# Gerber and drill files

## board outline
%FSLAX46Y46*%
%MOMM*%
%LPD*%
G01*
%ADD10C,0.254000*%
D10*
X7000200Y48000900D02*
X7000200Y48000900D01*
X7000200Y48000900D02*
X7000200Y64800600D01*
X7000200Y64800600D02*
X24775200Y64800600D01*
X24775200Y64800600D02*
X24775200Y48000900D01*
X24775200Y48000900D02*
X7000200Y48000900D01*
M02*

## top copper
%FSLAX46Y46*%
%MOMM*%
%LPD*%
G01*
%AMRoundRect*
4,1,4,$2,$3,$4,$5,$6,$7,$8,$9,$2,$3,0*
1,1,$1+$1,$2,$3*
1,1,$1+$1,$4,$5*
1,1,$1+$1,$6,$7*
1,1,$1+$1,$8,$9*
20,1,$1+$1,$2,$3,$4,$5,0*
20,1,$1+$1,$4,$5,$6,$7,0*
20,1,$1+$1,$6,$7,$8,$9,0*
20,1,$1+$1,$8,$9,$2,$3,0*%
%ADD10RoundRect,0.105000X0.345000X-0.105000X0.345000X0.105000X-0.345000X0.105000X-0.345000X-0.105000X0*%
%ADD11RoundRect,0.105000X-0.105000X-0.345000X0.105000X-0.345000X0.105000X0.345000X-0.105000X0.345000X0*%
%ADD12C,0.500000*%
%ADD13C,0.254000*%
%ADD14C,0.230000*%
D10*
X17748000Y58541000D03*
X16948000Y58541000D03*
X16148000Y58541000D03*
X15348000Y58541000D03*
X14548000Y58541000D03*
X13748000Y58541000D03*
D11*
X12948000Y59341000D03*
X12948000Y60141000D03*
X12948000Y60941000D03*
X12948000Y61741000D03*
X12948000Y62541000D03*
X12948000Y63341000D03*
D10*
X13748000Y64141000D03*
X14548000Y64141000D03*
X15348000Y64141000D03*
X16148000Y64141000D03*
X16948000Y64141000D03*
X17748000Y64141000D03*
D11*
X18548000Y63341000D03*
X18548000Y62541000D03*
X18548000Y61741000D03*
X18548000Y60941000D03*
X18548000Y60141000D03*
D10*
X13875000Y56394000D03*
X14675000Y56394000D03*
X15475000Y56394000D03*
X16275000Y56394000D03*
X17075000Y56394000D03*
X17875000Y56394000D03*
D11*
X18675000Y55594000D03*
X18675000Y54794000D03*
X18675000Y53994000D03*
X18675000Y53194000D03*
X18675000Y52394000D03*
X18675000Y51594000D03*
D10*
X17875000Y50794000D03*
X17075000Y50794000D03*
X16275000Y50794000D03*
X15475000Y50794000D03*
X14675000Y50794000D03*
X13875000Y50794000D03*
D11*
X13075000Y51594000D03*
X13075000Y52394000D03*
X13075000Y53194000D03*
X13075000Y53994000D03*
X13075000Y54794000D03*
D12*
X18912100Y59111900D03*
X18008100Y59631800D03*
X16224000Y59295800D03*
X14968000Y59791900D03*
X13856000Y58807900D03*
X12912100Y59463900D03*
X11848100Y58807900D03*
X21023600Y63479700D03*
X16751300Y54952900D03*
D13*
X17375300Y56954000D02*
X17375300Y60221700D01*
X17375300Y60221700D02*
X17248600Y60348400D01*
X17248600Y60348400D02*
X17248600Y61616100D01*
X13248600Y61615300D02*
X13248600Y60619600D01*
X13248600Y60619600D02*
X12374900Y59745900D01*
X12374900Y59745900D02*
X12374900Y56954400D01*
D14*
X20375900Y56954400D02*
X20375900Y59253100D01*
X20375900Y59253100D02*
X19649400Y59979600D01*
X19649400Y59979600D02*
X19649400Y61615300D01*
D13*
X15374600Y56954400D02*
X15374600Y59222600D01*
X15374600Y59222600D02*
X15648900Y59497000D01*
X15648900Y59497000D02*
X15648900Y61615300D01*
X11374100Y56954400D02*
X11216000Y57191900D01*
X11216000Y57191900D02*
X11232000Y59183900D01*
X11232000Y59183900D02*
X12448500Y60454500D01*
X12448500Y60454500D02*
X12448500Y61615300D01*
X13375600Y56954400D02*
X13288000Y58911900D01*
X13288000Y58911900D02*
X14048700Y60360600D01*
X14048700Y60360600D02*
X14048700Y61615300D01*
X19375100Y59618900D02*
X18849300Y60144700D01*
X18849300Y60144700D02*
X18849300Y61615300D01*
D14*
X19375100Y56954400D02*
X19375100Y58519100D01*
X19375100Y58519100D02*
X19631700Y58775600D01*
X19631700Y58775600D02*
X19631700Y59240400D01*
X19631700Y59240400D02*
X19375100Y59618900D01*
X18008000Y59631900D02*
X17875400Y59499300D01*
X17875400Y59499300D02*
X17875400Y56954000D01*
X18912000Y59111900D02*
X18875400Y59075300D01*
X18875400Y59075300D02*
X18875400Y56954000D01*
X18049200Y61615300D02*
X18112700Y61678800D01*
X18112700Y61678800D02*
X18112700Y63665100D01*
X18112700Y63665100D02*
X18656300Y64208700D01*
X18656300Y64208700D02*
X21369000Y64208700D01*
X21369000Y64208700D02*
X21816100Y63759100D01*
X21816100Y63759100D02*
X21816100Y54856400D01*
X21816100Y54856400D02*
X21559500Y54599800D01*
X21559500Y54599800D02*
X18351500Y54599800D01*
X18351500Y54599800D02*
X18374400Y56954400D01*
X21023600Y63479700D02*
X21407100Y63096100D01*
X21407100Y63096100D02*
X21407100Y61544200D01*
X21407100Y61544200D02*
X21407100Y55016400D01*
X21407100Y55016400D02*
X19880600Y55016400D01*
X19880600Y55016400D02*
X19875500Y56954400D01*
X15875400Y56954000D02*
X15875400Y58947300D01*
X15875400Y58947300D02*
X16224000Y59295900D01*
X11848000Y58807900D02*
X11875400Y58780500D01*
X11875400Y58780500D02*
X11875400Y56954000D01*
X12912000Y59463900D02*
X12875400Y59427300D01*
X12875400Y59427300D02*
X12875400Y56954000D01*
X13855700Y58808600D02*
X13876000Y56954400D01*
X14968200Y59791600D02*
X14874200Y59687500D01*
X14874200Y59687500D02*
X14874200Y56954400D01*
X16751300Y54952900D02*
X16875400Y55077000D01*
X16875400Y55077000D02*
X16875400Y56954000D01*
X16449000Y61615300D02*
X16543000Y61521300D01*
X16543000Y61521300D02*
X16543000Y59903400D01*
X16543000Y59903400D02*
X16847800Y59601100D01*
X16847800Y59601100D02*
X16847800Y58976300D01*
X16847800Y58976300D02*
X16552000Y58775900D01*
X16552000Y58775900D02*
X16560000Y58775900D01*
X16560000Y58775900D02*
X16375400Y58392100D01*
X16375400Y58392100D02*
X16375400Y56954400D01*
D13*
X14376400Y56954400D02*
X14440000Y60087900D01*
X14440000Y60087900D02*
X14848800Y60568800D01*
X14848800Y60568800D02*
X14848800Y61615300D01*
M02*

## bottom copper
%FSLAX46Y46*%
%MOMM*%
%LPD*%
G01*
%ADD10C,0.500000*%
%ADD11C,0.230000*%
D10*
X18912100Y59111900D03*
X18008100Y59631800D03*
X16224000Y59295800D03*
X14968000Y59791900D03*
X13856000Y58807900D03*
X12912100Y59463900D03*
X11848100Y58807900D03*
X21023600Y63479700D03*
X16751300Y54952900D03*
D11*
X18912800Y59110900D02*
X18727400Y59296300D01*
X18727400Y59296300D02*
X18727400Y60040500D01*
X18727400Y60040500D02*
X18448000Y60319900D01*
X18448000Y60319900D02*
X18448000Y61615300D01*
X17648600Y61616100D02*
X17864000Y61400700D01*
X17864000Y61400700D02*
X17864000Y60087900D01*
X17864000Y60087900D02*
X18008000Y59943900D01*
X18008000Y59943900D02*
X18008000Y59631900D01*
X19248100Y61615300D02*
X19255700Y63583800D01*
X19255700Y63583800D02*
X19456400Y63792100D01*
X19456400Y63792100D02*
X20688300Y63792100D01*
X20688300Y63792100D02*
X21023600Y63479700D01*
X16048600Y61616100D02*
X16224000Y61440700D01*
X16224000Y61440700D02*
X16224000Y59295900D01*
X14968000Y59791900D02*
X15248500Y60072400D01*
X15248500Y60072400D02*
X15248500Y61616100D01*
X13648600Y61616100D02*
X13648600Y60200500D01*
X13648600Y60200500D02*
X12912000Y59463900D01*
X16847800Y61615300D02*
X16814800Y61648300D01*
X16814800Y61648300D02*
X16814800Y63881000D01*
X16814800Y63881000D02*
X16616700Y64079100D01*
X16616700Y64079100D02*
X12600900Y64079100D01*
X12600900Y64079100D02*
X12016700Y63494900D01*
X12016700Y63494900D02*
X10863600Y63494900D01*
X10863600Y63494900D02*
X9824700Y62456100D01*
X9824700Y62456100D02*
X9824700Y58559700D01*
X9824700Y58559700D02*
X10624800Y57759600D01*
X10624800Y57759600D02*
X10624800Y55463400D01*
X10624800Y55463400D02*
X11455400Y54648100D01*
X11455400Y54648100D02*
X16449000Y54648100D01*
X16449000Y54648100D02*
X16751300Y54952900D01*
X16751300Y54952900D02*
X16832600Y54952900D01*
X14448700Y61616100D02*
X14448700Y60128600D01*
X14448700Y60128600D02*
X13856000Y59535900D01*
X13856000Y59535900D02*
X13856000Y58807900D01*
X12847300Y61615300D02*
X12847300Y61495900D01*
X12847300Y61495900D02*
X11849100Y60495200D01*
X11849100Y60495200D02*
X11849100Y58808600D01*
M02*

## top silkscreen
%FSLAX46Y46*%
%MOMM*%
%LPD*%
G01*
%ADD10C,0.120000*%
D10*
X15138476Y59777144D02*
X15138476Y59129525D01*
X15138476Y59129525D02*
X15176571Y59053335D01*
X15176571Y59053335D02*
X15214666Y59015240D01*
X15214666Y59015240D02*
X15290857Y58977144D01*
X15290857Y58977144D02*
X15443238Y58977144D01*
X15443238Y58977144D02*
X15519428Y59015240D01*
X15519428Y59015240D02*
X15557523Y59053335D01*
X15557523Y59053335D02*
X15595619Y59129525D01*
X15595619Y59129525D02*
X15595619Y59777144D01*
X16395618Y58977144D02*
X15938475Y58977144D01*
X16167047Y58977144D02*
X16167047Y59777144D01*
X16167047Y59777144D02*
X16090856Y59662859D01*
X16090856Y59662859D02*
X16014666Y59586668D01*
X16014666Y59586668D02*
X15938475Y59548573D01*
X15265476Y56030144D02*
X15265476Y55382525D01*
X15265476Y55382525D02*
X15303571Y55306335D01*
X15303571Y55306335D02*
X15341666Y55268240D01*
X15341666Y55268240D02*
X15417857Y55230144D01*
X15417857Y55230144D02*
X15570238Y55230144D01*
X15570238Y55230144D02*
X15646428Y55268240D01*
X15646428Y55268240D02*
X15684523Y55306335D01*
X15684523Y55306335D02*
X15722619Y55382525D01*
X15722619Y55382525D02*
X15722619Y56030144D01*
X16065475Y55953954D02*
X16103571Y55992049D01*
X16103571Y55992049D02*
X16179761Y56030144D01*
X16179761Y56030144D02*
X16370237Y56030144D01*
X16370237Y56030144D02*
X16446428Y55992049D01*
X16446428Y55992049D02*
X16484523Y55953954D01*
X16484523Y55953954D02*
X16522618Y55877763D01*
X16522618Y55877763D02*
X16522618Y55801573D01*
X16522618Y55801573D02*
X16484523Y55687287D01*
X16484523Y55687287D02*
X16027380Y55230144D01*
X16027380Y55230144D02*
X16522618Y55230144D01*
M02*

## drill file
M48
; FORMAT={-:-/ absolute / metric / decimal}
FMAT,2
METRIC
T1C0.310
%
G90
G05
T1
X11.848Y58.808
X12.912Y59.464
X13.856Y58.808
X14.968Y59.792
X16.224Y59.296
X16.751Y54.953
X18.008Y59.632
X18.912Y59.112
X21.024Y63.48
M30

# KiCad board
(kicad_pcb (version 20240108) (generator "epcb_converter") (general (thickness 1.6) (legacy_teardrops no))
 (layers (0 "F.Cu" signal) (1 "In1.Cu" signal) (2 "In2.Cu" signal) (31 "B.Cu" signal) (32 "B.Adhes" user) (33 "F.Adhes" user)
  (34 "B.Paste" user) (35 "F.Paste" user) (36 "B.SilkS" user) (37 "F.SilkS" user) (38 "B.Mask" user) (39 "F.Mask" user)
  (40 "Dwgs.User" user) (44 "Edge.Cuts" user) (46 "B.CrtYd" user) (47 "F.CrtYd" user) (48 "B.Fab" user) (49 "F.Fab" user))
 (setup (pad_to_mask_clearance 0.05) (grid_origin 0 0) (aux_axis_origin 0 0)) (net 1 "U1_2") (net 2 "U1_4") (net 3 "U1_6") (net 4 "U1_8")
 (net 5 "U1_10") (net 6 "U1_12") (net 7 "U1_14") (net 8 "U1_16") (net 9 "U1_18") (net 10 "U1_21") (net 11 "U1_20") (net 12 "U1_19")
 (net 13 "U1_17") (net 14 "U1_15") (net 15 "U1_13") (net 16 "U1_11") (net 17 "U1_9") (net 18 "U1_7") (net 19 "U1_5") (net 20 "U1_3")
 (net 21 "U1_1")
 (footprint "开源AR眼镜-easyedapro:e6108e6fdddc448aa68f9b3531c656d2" (layer "F.Cu") (at 15.748 -61.340999999999994 180.0000)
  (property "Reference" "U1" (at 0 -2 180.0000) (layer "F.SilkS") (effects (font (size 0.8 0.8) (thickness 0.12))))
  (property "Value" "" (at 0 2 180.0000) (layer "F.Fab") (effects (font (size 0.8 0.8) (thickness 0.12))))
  (pad "2" smd roundrect (at -2.0000 -2.8000 90.0000) (size 0.4200 0.9000) (layers "F.Cu" "F.Paste" "F.Mask") (roundrect_rratio 0.25)
   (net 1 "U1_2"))
  (pad "4" smd roundrect (at -1.2000 -2.8000 90.0000) (size 0.4200 0.9000) (layers "F.Cu" "F.Paste" "F.Mask") (roundrect_rratio 0.25)
   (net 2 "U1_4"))
  (pad "6" smd roundrect (at -0.4000 -2.8000 90.0000) (size 0.4200 0.9000) (layers "F.Cu" "F.Paste" "F.Mask") (roundrect_rratio 0.25)
   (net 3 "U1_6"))
  (pad "8" smd roundrect (at 0.4000 -2.8000 90.0000) (size 0.4200 0.9000) (layers "F.Cu" "F.Paste" "F.Mask") (roundrect_rratio 0.25)
   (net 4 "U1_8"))
  (pad "10" smd roundrect (at 1.2000 -2.8000 90.0000) (size 0.4200 0.9000) (layers "F.Cu" "F.Paste" "F.Mask") (roundrect_rratio 0.25)
   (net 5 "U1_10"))
  (pad "12" smd roundrect (at 2.0000 -2.8000 90.0000) (size 0.4200 0.9000) (layers "F.Cu" "F.Paste" "F.Mask") (roundrect_rratio 0.25)
   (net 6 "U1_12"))
  (pad "14" smd roundrect (at 2.8000 -2.0000 0.0000) (size 0.4200 0.9000) (layers "F.Cu" "F.Paste" "F.Mask") (roundrect_rratio 0.25)
   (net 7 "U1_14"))
  (pad "16" smd roundrect (at 2.8000 -1.2000 0.0000) (size 0.4200 0.9000) (layers "F.Cu" "F.Paste" "F.Mask") (roundrect_rratio 0.25)
   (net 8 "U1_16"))
  (pad "18" smd roundrect (at 2.8000 -0.4000 0.0000) (size 0.4200 0.9000) (layers "F.Cu" "F.Paste" "F.Mask") (roundrect_rratio 0.25)
   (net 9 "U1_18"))
  (pad "21" smd roundrect (at 2.8000 0.4000 0.0000) (size 0.4200 0.9000) (layers "F.Cu" "F.Paste" "F.Mask") (roundrect_rratio 0.25)
   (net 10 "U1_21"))
  (pad "20" smd roundrect (at 2.8000 1.2000 0.0000) (size 0.4200 0.9000) (layers "F.Cu" "F.Paste" "F.Mask") (roundrect_rratio 0.25)
   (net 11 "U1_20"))
  (pad "19" smd roundrect (at 2.8000 2.0000 0.0000) (size 0.4200 0.9000) (layers "F.Cu" "F.Paste" "F.Mask") (roundrect_rratio 0.25)
   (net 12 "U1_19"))
  (pad "17" smd roundrect (at 2.0000 2.8000 90.0000) (size 0.4200 0.9000) (layers "F.Cu" "F.Paste" "F.Mask") (roundrect_rratio 0.25)
   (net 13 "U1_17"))
  (pad "15" smd roundrect (at 1.2000 2.8000 90.0000) (size 0.4200 0.9000) (layers "F.Cu" "F.Paste" "F.Mask") (roundrect_rratio 0.25)
   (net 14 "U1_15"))
  (pad "13" smd roundrect (at 0.4000 2.8000 90.0000) (size 0.4200 0.9000) (layers "F.Cu" "F.Paste" "F.Mask") (roundrect_rratio 0.25)
   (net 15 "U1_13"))
  (pad "11" smd roundrect (at -0.4000 2.8000 90.0000) (size 0.4200 0.9000) (layers "F.Cu" "F.Paste" "F.Mask") (roundrect_rratio 0.25)
   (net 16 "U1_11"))
  (pad "9" smd roundrect (at -1.2000 2.8000 90.0000) (size 0.4200 0.9000) (layers "F.Cu" "F.Paste" "F.Mask") (roundrect_rratio 0.25)
   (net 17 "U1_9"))
  (pad "7" smd roundrect (at -2.0000 2.8000 90.0000) (size 0.4200 0.9000) (layers "F.Cu" "F.Paste" "F.Mask") (roundrect_rratio 0.25)
   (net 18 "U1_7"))
  (pad "5" smd roundrect (at -2.8000 2.0000 0.0000) (size 0.4200 0.9000) (layers "F.Cu" "F.Paste" "F.Mask") (roundrect_rratio 0.25)
   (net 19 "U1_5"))
  (pad "3" smd roundrect (at -2.8000 1.2000 0.0000) (size 0.4200 0.9000) (layers "F.Cu" "F.Paste" "F.Mask") (roundrect_rratio 0.25)
   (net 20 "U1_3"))
  (pad "1" smd roundrect (at -2.8000 0.4000 0.0000) (size 0.4200 0.9000) (layers "F.Cu" "F.Paste" "F.Mask") (roundrect_rratio 0.25)
   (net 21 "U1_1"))
  (pad "22" smd roundrect (at -2.8000 -0.4000 0.0000) (size 0.4200 0.9000) (layers "F.Cu" "F.Paste" "F.Mask") (roundrect_rratio 0.25)
   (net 10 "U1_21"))
  (pad "23" smd roundrect (at -2.8000 -1.2000 0.0000) (size 0.4200 0.9000) (layers "F.Cu" "F.Paste" "F.Mask") (roundrect_rratio 0.25)
   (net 11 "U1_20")))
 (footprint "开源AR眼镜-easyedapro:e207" (layer "F.Cu") (at 15.875 -53.594 0.0000)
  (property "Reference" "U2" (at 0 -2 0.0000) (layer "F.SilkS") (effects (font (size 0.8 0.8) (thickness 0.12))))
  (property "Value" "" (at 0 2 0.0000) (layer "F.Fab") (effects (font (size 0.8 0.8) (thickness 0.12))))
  (pad "1" smd roundrect (at -2.0000 -2.8000 90.0000) (size 0.4200 0.9000) (layers "F.Cu" "F.Paste" "F.Mask") (roundrect_rratio 0.25)
   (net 21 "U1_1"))
  (pad "2" smd roundrect (at -1.2000 -2.8000 90.0000) (size 0.4200 0.9000) (layers "F.Cu" "F.Paste" "F.Mask") (roundrect_rratio 0.25)
   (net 1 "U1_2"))
  (pad "3" smd roundrect (at -0.4000 -2.8000 90.0000) (size 0.4200 0.9000) (layers "F.Cu" "F.Paste" "F.Mask") (roundrect_rratio 0.25)
   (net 20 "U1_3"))
  (pad "4" smd roundrect (at 0.4000 -2.8000 90.0000) (size 0.4200 0.9000) (layers "F.Cu" "F.Paste" "F.Mask") (roundrect_rratio 0.25)
   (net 2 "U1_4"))
  (pad "5" smd roundrect (at 1.2000 -2.8000 90.0000) (size 0.4200 0.9000) (layers "F.Cu" "F.Paste" "F.Mask") (roundrect_rratio 0.25)
   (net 19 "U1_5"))
  (pad "6" smd roundrect (at 2.0000 -2.8000 90.0000) (size 0.4200 0.9000) (layers "F.Cu" "F.Paste" "F.Mask") (roundrect_rratio 0.25)
   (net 3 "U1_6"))
  (pad "7" smd roundrect (at 2.8000 -2.0000 0.0000) (size 0.4200 0.9000) (layers "F.Cu" "F.Paste" "F.Mask") (roundrect_rratio 0.25)
   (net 18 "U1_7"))
  (pad "8" smd roundrect (at 2.8000 -1.2000 0.0000) (size 0.4200 0.9000) (layers "F.Cu" "F.Paste" "F.Mask") (roundrect_rratio 0.25)
   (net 4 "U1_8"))
  (pad "9" smd roundrect (at 2.8000 -0.4000 0.0000) (size 0.4200 0.9000) (layers "F.Cu" "F.Paste" "F.Mask") (roundrect_rratio 0.25)
   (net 17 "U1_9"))
  (pad "10" smd roundrect (at 2.8000 0.4000 0.0000) (size 0.4200 0.9000) (layers "F.Cu" "F.Paste" "F.Mask") (roundrect_rratio 0.25)
   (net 5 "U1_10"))
  (pad "11" smd roundrect (at 2.8000 1.2000 0.0000) (size 0.4200 0.9000) (layers "F.Cu" "F.Paste" "F.Mask") (roundrect_rratio 0.25)
   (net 16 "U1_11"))
  (pad "12" smd roundrect (at 2.8000 2.0000 0.0000) (size 0.4200 0.9000) (layers "F.Cu" "F.Paste" "F.Mask") (roundrect_rratio 0.25)
   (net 6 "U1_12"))
  (pad "13" smd roundrect (at 2.0000 2.8000 90.0000) (size 0.4200 0.9000) (layers "F.Cu" "F.Paste" "F.Mask") (roundrect_rratio 0.25)
   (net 15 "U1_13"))
  (pad "14" smd roundrect (at 1.2000 2.8000 90.0000) (size 0.4200 0.9000) (layers "F.Cu" "F.Paste" "F.Mask") (roundrect_rratio 0.25)
   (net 7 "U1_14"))
  (pad "15" smd roundrect (at 0.4000 2.8000 90.0000) (size 0.4200 0.9000) (layers "F.Cu" "F.Paste" "F.Mask") (roundrect_rratio 0.25)
   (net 14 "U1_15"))
  (pad "16" smd roundrect (at -0.4000 2.8000 90.0000) (size 0.4200 0.9000) (layers "F.Cu" "F.Paste" "F.Mask") (roundrect_rratio 0.25)
   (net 8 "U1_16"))
  (pad "17" smd roundrect (at -1.2000 2.8000 90.0000) (size 0.4200 0.9000) (layers "F.Cu" "F.Paste" "F.Mask") (roundrect_rratio 0.25)
   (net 13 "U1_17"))
  (pad "18" smd roundrect (at -2.0000 2.8000 90.0000) (size 0.4200 0.9000) (layers "F.Cu" "F.Paste" "F.Mask") (roundrect_rratio 0.25)
   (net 9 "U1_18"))
  (pad "19" smd roundrect (at -2.8000 2.0000 0.0000) (size 0.4200 0.9000) (layers "F.Cu" "F.Paste" "F.Mask") (roundrect_rratio 0.25)
   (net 12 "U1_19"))
  (pad "20" smd roundrect (at -2.8000 1.2000 0.0000) (size 0.4200 0.9000) (layers "F.Cu" "F.Paste" "F.Mask") (roundrect_rratio 0.25)
   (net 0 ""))
  (pad "22" smd roundrect (at -2.8000 0.4000 0.0000) (size 0.4200 0.9000) (layers "F.Cu" "F.Paste" "F.Mask") (roundrect_rratio 0.25)
   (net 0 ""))
  (pad "23" smd roundrect (at -2.8000 -0.4000 0.0000) (size 0.4200 0.9000) (layers "F.Cu" "F.Paste" "F.Mask") (roundrect_rratio 0.25)
   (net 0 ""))
  (pad "21" smd roundrect (at -2.8000 -1.2000 0.0000) (size 0.4200 0.9000) (layers "F.Cu" "F.Paste" "F.Mask") (roundrect_rratio 0.25)
   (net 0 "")))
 (via (at 18.9121 -59.1119) (size 0.5000) (drill 0.3100) (layers "F.Cu" "B.Cu") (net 2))
 (via (at 18.0081 -59.6318) (size 0.5000) (drill 0.3100) (layers "F.Cu" "B.Cu") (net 3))
 (via (at 16.2240 -59.2958) (size 0.5000) (drill 0.3100) (layers "F.Cu" "B.Cu") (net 5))
 (via (at 14.9680 -59.7919) (size 0.5000) (drill 0.3100) (layers "F.Cu" "B.Cu") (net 6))
 (via (at 13.8560 -58.8079) (size 0.5000) (drill 0.3100) (layers "F.Cu" "B.Cu") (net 7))
 (via (at 12.9121 -59.4639) (size 0.5000) (drill 0.3100) (layers "F.Cu" "B.Cu") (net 8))
 (via (at 11.8481 -58.8079) (size 0.5000) (drill 0.3100) (layers "F.Cu" "B.Cu") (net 9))
 (via (at 21.0236 -63.4797) (size 0.5000) (drill 0.3100) (layers "F.Cu" "B.Cu") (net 1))
 (via (at 16.7513 -54.9529) (size 0.5000) (drill 0.3100) (layers "F.Cu" "B.Cu") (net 4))
 (segment (start 17.3753 -56.9540) (end 17.3753 -60.2217) (width 0.2540) (layer "F.Cu") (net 18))
 (segment (start 17.3753 -60.2217) (end 17.2486 -60.3484) (width 0.2540) (layer "F.Cu") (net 18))
 (segment (start 17.2486 -60.3484) (end 17.2486 -61.6161) (width 0.2540) (layer "F.Cu") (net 18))
 (segment (start 13.2486 -61.6153) (end 13.2486 -60.6196) (width 0.2540) (layer "F.Cu") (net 13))
 (segment (start 13.2486 -60.6196) (end 12.3749 -59.7459) (width 0.2540) (layer "F.Cu") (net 13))
 (segment (start 12.3749 -59.7459) (end 12.3749 -56.9544) (width 0.2540) (layer "F.Cu") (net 13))
 (segment (start 20.3759 -56.9544) (end 20.3759 -59.2531) (width 0.2300) (layer "F.Cu") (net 21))
 (segment (start 20.3759 -59.2531) (end 19.6494 -59.9796) (width 0.2300) (layer "F.Cu") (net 21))
 (segment (start 19.6494 -59.9796) (end 19.6494 -61.6153) (width 0.2300) (layer "F.Cu") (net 21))
 (segment (start 15.3746 -56.9544) (end 15.3746 -59.2226) (width 0.2540) (layer "F.Cu") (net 16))
 (segment (start 15.3746 -59.2226) (end 15.6489 -59.4970) (width 0.2540) (layer "F.Cu") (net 16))
 (segment (start 15.6489 -59.4970) (end 15.6489 -61.6153) (width 0.2540) (layer "F.Cu") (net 16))
 (segment (start 11.3741 -56.9544) (end 11.2160 -57.1919) (width 0.2540) (layer "F.Cu") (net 12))
 (segment (start 11.2160 -57.1919) (end 11.2320 -59.1839) (width 0.2540) (layer "F.Cu") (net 12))
 (segment (start 11.2320 -59.1839) (end 12.4485 -60.4545) (width 0.2540) (layer "F.Cu") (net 12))
 (segment (start 12.4485 -60.4545) (end 12.4485 -61.6153) (width 0.2540) (layer "F.Cu") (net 12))
 (segment (start 13.3756 -56.9544) (end 13.2880 -58.9119) (width 0.2540) (layer "F.Cu") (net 14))
 (segment (start 13.2880 -58.9119) (end 14.0487 -60.3606) (width 0.2540) (layer "F.Cu") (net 14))
 (segment (start 14.0487 -60.3606) (end 14.0487 -61.6153) (width 0.2540) (layer "F.Cu") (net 14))
 (segment (start 19.3751 -59.6189) (end 18.8493 -60.1447) (width 0.2540) (layer "F.Cu") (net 20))
 (segment (start 18.8493 -60.1447) (end 18.8493 -61.6153) (width 0.2540) (layer "F.Cu") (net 20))
 (segment (start 19.3751 -56.9544) (end 19.3751 -58.5191) (width 0.2300) (layer "F.Cu") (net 20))
 (segment (start 19.3751 -58.5191) (end 19.6317 -58.7756) (width 0.2300) (layer "F.Cu") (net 20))
 (segment (start 19.6317 -58.7756) (end 19.6317 -59.2404) (width 0.2300) (layer "F.Cu") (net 20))
 (segment (start 19.6317 -59.2404) (end 19.3751 -59.6189) (width 0.2300) (layer "F.Cu") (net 20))
 (segment (start 18.0080 -59.6319) (end 17.8754 -59.4993) (width 0.2300) (layer "F.Cu") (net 3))
 (segment (start 17.8754 -59.4993) (end 17.8754 -56.9540) (width 0.2300) (layer "F.Cu") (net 3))
 (segment (start 18.9120 -59.1119) (end 18.8754 -59.0753) (width 0.2300) (layer "F.Cu") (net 2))
 (segment (start 18.8754 -59.0753) (end 18.8754 -56.9540) (width 0.2300) (layer "F.Cu") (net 2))
 (segment (start 18.0492 -61.6153) (end 18.1127 -61.6788) (width 0.2300) (layer "F.Cu") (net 19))
 (segment (start 18.1127 -61.6788) (end 18.1127 -63.6651) (width 0.2300) (layer "F.Cu") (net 19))
 (segment (start 18.1127 -63.6651) (end 18.6563 -64.2087) (width 0.2300) (layer "F.Cu") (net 19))
 (segment (start 18.6563 -64.2087) (end 21.3690 -64.2087) (width 0.2300) (layer "F.Cu") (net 19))
 (segment (start 21.3690 -64.2087) (end 21.8161 -63.7591) (width 0.2300) (layer "F.Cu") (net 19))
 (segment (start 21.8161 -63.7591) (end 21.8161 -54.8564) (width 0.2300) (layer "F.Cu") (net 19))
 (segment (start 21.8161 -54.8564) (end 21.5595 -54.5998) (width 0.2300) (layer "F.Cu") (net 19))
 (segment (start 21.5595 -54.5998) (end 18.3515 -54.5998) (width 0.2300) (layer "F.Cu") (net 19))
 (segment (start 18.3515 -54.5998) (end 18.3744 -56.9544) (width 0.2300) (layer "F.Cu") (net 19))
 (segment (start 21.0236 -63.4797) (end 21.4071 -63.0961) (width 0.2300) (layer "F.Cu") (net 1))
 (segment (start 21.4071 -63.0961) (end 21.4071 -61.5442) (width 0.2300) (layer "F.Cu") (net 1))
 (segment (start 21.4071 -61.5442) (end 21.4071 -55.0164) (width 0.2300) (layer "F.Cu") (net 1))
 (segment (start 21.4071 -55.0164) (end 19.8806 -55.0164) (width 0.2300) (layer "F.Cu") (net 1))
 (segment (start 19.8806 -55.0164) (end 19.8755 -56.9544) (width 0.2300) (layer "F.Cu") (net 1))
 (segment (start 15.8754 -56.9540) (end 15.8754 -58.9473) (width 0.2300) (layer "F.Cu") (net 5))
 (segment (start 15.8754 -58.9473) (end 16.2240 -59.2959) (width 0.2300) (layer "F.Cu") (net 5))
 (segment (start 11.8480 -58.8079) (end 11.8754 -58.7805) (width 0.2300) (layer "F.Cu") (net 9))
 (segment (start 11.8754 -58.7805) (end 11.8754 -56.9540) (width 0.2300) (layer "F.Cu") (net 9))
 (segment (start 12.9120 -59.4639) (end 12.8754 -59.4273) (width 0.2300) (layer "F.Cu") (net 8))
 (segment (start 12.8754 -59.4273) (end 12.8754 -56.9540) (width 0.2300) (layer "F.Cu") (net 8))
 (segment (start 13.8557 -58.8086) (end 13.8760 -56.9544) (width 0.2300) (layer "F.Cu") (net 7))
 (segment (start 14.9682 -59.7916) (end 14.8742 -59.6875) (width 0.2300) (layer "F.Cu") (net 6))
 (segment (start 14.8742 -59.6875) (end 14.8742 -56.9544) (width 0.2300) (layer "F.Cu") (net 6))
 (segment (start 16.7513 -54.9529) (end 16.8754 -55.0770) (width 0.2300) (layer "F.Cu") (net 4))
 (segment (start 16.8754 -55.0770) (end 16.8754 -56.9540) (width 0.2300) (layer "F.Cu") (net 4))
 (segment (start 16.4490 -61.6153) (end 16.5430 -61.5213) (width 0.2300) (layer "F.Cu") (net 17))
 (segment (start 16.5430 -61.5213) (end 16.5430 -59.9034) (width 0.2300) (layer "F.Cu") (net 17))
 (segment (start 16.5430 -59.9034) (end 16.8478 -59.6011) (width 0.2300) (layer "F.Cu") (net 17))
 (segment (start 16.8478 -59.6011) (end 16.8478 -58.9763) (width 0.2300) (layer "F.Cu") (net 17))
 (segment (start 16.8478 -58.9763) (end 16.5520 -58.7759) (width 0.2300) (layer "F.Cu") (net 17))
 (segment (start 16.5520 -58.7759) (end 16.5600 -58.7759) (width 0.2300) (layer "F.Cu") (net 17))
 (segment (start 16.5600 -58.7759) (end 16.3754 -58.3921) (width 0.2300) (layer "F.Cu") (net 17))
 (segment (start 16.3754 -58.3921) (end 16.3754 -56.9544) (width 0.2300) (layer "F.Cu") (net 17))
 (segment (start 14.3764 -56.9544) (end 14.4400 -60.0879) (width 0.2540) (layer "F.Cu") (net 15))
 (segment (start 14.4400 -60.0879) (end 14.8488 -60.5688) (width 0.2540) (layer "F.Cu") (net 15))
 (segment (start 14.8488 -60.5688) (end 14.8488 -61.6153) (width 0.2540) (layer "F.Cu") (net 15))
 (segment (start 18.9128 -59.1109) (end 18.7274 -59.2963) (width 0.2300) (layer "B.Cu") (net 2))
 (segment (start 18.7274 -59.2963) (end 18.7274 -60.0405) (width 0.2300) (layer "B.Cu") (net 2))
 (segment (start 18.7274 -60.0405) (end 18.4480 -60.3199) (width 0.2300) (layer "B.Cu") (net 2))
 (segment (start 18.4480 -60.3199) (end 18.4480 -61.6153) (width 0.2300) (layer "B.Cu") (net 2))
 (segment (start 17.6486 -61.6161) (end 17.8640 -61.4007) (width 0.2300) (layer "B.Cu") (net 3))
 (segment (start 17.8640 -61.4007) (end 17.8640 -60.0879) (width 0.2300) (layer "B.Cu") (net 3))
 (segment (start 17.8640 -60.0879) (end 18.0080 -59.9439) (width 0.2300) (layer "B.Cu") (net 3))
 (segment (start 18.0080 -59.9439) (end 18.0080 -59.6319) (width 0.2300) (layer "B.Cu") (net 3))
 (segment (start 19.2481 -61.6153) (end 19.2557 -63.5838) (width 0.2300) (layer "B.Cu") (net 1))
 (segment (start 19.2557 -63.5838) (end 19.4564 -63.7921) (width 0.2300) (layer "B.Cu") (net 1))
 (segment (start 19.4564 -63.7921) (end 20.6883 -63.7921) (width 0.2300) (layer "B.Cu") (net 1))
 (segment (start 20.6883 -63.7921) (end 21.0236 -63.4797) (width 0.2300) (layer "B.Cu") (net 1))
 (segment (start 16.0486 -61.6161) (end 16.2240 -61.4407) (width 0.2300) (layer "B.Cu") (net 5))
 (segment (start 16.2240 -61.4407) (end 16.2240 -59.2959) (width 0.2300) (layer "B.Cu") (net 5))
 (segment (start 14.9680 -59.7919) (end 15.2485 -60.0724) (width 0.2300) (layer "B.Cu") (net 6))
 (segment (start 15.2485 -60.0724) (end 15.2485 -61.6161) (width 0.2300) (layer "B.Cu") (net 6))
 (segment (start 13.6486 -61.6161) (end 13.6486 -60.2005) (width 0.2300) (layer "B.Cu") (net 8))
 (segment (start 13.6486 -60.2005) (end 12.9120 -59.4639) (width 0.2300) (layer "B.Cu") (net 8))
 (segment (start 16.8478 -61.6153) (end 16.8148 -61.6483) (width 0.2300) (layer "B.Cu") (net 4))
 (segment (start 16.8148 -61.6483) (end 16.8148 -63.8810) (width 0.2300) (layer "B.Cu") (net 4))
 (segment (start 16.8148 -63.8810) (end 16.6167 -64.0791) (width 0.2300) (layer "B.Cu") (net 4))
 (segment (start 16.6167 -64.0791) (end 12.6009 -64.0791) (width 0.2300) (layer "B.Cu") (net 4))
 (segment (start 12.6009 -64.0791) (end 12.0167 -63.4949) (width 0.2300) (layer "B.Cu") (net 4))
 (segment (start 12.0167 -63.4949) (end 10.8636 -63.4949) (width 0.2300) (layer "B.Cu") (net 4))
 (segment (start 10.8636 -63.4949) (end 9.8247 -62.4561) (width 0.2300) (layer "B.Cu") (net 4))
 (segment (start 9.8247 -62.4561) (end 9.8247 -58.5597) (width 0.2300) (layer "B.Cu") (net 4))
 (segment (start 9.8247 -58.5597) (end 10.6248 -57.7596) (width 0.2300) (layer "B.Cu") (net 4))
 (segment (start 10.6248 -57.7596) (end 10.6248 -55.4634) (width 0.2300) (layer "B.Cu") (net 4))
 (segment (start 10.6248 -55.4634) (end 11.4554 -54.6481) (width 0.2300) (layer "B.Cu") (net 4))
 (segment (start 11.4554 -54.6481) (end 16.4490 -54.6481) (width 0.2300) (layer "B.Cu") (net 4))
 (segment (start 16.4490 -54.6481) (end 16.7513 -54.9529) (width 0.2300) (layer "B.Cu") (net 4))
 (segment (start 16.7513 -54.9529) (end 16.8326 -54.9529) (width 0.2300) (layer "B.Cu") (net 4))
 (segment (start 14.4487 -61.6161) (end 14.4487 -60.1286) (width 0.2300) (layer "B.Cu") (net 7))
 (segment (start 14.4487 -60.1286) (end 13.8560 -59.5359) (width 0.2300) (layer "B.Cu") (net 7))
 (segment (start 13.8560 -59.5359) (end 13.8560 -58.8079) (width 0.2300) (layer "B.Cu") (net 7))
 (segment (start 12.8473 -61.6153) (end 12.8473 -61.4959) (width 0.2300) (layer "B.Cu") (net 9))
 (segment (start 12.8473 -61.4959) (end 11.8491 -60.4952) (width 0.2300) (layer "B.Cu") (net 9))
 (segment (start 11.8491 -60.4952) (end 11.8491 -58.8086) (width 0.2300) (layer "B.Cu") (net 9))
 (segment (start 12.7840 -61.4319) (end 12.7840 -61.4319) (width 0.1270) (layer "B.Mask") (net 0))
 (segment (start 12.7840 -61.4319) (end 11.8880 -60.5359) (width 0.1270) (layer "B.Mask") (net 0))
 (segment (start 11.8880 -60.5359) (end 11.8880 -60.5359) (width 0.1270) (layer "B.Mask") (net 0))
 (segment (start 11.8880 -60.5359) (end 11.8880 -60.1919) (width 0.1270) (layer "B.Mask") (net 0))
 (segment (start 11.8880 -60.1919) (end 11.8880 -60.1919) (width 0.1270) (layer "B.Mask") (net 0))
 (segment (start 11.8880 -60.1919) (end 11.8880 -58.9199) (width 0.1270) (layer "B.Mask") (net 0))
 (segment (start 12.9280 -59.5119) (end 12.9280 -59.5119) (width 0.1270) (layer "B.Mask") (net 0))
 (segment (start 12.9280 -59.5119) (end 13.6640 -60.2479) (width 0.1270) (layer "B.Mask") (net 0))
 (segment (start 13.6640 -60.2479) (end 13.6640 -60.2479) (width 0.1270) (layer "B.Mask") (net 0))
 (segment (start 13.6640 -60.2479) (end 13.6640 -61.0959) (width 0.1270) (layer "B.Mask") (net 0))
 (segment (start 13.8400 -58.7679) (end 13.8400 -58.7679) (width 0.1270) (layer "B.Mask") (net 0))
 (segment (start 13.8400 -58.7679) (end 13.8640 -58.7919) (width 0.1270) (layer "B.Mask") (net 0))
 (segment (start 13.8640 -58.7919) (end 13.8640 -58.7919) (width 0.1270) (layer "B.Mask") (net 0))
 (segment (start 13.8640 -58.7919) (end 13.8640 -59.5279) (width 0.1270) (layer "B.Mask") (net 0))
 (segment (start 13.8640 -59.5279) (end 13.8640 -59.5279) (width 0.1270) (layer "B.Mask") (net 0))
 (segment (start 13.8640 -59.5279) (end 14.4560 -60.1199) (width 0.1270) (layer "B.Mask") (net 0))
 (segment (start 14.4560 -60.1199) (end 14.4560 -60.1199) (width 0.1270) (layer "B.Mask") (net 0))
 (segment (start 14.4560 -60.1199) (end 14.4560 -60.8239) (width 0.1270) (layer "B.Mask") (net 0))
 (segment (start 14.9440 -59.7999) (end 14.9440 -59.7999) (width 0.1270) (layer "B.Mask") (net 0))
 (segment (start 14.9440 -59.7999) (end 15.2160 -60.0719) (width 0.1270) (layer "B.Mask") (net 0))
 (segment (start 15.2160 -60.0719) (end 15.2160 -60.0719) (width 0.1270) (layer "B.Mask") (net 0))
 (segment (start 15.2160 -60.0719) (end 15.2240 -60.0719) (width 0.1270) (layer "B.Mask") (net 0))
 (segment (start 15.2240 -60.0719) (end 15.2240 -60.0719) (width 0.1270) (layer "B.Mask") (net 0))
 (segment (start 15.2240 -60.0719) (end 15.2640 -60.1119) (width 0.1270) (layer "B.Mask") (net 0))
 (segment (start 15.2640 -60.1119) (end 15.2640 -60.1119) (width 0.1270) (layer "B.Mask") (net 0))
 (segment (start 15.2640 -60.1119) (end 15.2640 -61.0959) (width 0.1270) (layer "B.Mask") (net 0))
 (segment (start 16.2000 -59.4719) (end 16.2000 -59.4719) (width 0.1270) (layer "B.Mask") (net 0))
 (segment (start 16.2000 -59.4719) (end 16.2240 -59.4959) (width 0.1270) (layer "B.Mask") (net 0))
 (segment (start 16.2240 -59.4959) (end 16.2240 -59.4959) (width 0.1270) (layer "B.Mask") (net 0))
 (segment (start 16.2240 -59.4959) (end 16.2240 -60.7199) (width 0.1270) (layer "B.Mask") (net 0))
 (segment (start 17.9440 -59.6959) (end 17.9440 -59.6959) (width 0.1270) (layer "B.Mask") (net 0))
 (segment (start 17.9440 -59.6959) (end 18.0160 -59.7679) (width 0.1270) (layer "B.Mask") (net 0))
 (segment (start 18.0160 -59.7679) (end 18.0160 -59.7679) (width 0.1270) (layer "B.Mask") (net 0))
 (segment (start 18.0160 -59.7679) (end 18.0160 -59.9119) (width 0.1270) (layer "B.Mask") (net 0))
 (segment (start 18.0160 -59.9119) (end 18.0160 -59.9119) (width 0.1270) (layer "B.Mask") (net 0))
 (segment (start 18.0160 -59.9119) (end 17.8640 -60.0639) (width 0.1270) (layer "B.Mask") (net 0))
 (segment (start 17.8640 -60.0639) (end 17.8640 -60.0639) (width 0.1270) (layer "B.Mask") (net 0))
 (segment (start 17.8640 -60.0639) (end 17.8640 -60.6079) (width 0.1270) (layer "B.Mask") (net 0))
 (segment (start 18.4640 -60.8879) (end 18.4640 -60.8879) (width 0.1270) (layer "B.Mask") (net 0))
 (segment (start 18.4640 -60.8879) (end 18.4640 -60.2879) (width 0.1270) (layer "B.Mask") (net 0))
 (segment (start 18.4640 -60.2879) (end 18.4640 -60.2879) (width 0.1270) (layer "B.Mask") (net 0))
 (segment (start 18.4640 -60.2879) (end 18.7600 -59.9919) (width 0.1270) (layer "B.Mask") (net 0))
 (segment (start 18.7600 -59.9919) (end 18.7600 -59.9919) (width 0.1270) (layer "B.Mask") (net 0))
 (segment (start 18.7600 -59.9919) (end 18.7600 -59.2319) (width 0.1270) (layer "B.Mask") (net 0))
 (segment (start 13.3909 -58.0568) (end 13.3909 -58.0568) (width 0.1270) (layer "F.Mask") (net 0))
 (segment (start 13.3909 -58.0568) (end 13.2969 -58.1508) (width 0.1270) (layer "F.Mask") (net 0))
 (segment (start 13.2969 -58.1508) (end 13.2969 -58.1508) (width 0.1270) (layer "F.Mask") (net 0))
 (segment (start 13.2969 -58.1508) (end 13.2969 -58.8797) (width 0.1270) (layer "F.Mask") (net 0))
 (segment (start 13.2969 -58.8797) (end 13.2969 -58.8797) (width 0.1270) (layer "F.Mask") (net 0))
 (segment (start 13.2969 -58.8797) (end 14.0310 -60.3758) (width 0.1270) (layer "F.Mask") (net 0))
 (segment (start 14.0310 -60.3758) (end 14.0310 -60.3758) (width 0.1270) (layer "F.Mask") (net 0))
 (segment (start 14.0310 -60.3758) (end 14.0487 -60.3910) (width 0.1270) (layer "F.Mask") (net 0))
 (segment (start 14.0487 -60.3910) (end 14.0487 -60.3910) (width 0.1270) (layer "F.Mask") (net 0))
 (segment (start 14.0487 -60.3910) (end 14.0487 -61.5747) (width 0.1270) (layer "F.Mask") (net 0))
 (segment (start 16.3347 -58.0949) (end 16.3347 -58.0949) (width 0.1270) (layer "F.Mask") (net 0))
 (segment (start 16.3347 -58.0949) (end 16.3601 -58.1203) (width 0.1270) (layer "F.Mask") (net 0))
 (segment (start 16.3601 -58.1203) (end 16.3601 -58.1203) (width 0.1270) (layer "F.Mask") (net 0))
 (segment (start 16.3601 -58.1203) (end 16.3601 -58.3667) (width 0.1270) (layer "F.Mask") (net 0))
 (segment (start 16.3601 -58.3667) (end 16.3601 -58.3667) (width 0.1270) (layer "F.Mask") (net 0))
 (segment (start 16.3601 -58.3667) (end 16.3678 -58.3768) (width 0.1270) (layer "F.Mask") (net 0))
 (segment (start 16.3678 -58.3768) (end 16.3678 -58.3768) (width 0.1270) (layer "F.Mask") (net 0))
 (segment (start 16.3678 -58.3768) (end 16.3678 -58.3667) (width 0.1270) (layer "F.Mask") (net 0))
 (segment (start 16.3678 -58.3667) (end 16.3678 -58.3667) (width 0.1270) (layer "F.Mask") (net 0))
 (segment (start 16.3678 -58.3667) (end 16.5532 -58.7680) (width 0.1270) (layer "F.Mask") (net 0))
 (segment (start 16.5532 -58.7680) (end 16.5532 -58.7680) (width 0.1270) (layer "F.Mask") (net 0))
 (segment (start 16.5532 -58.7680) (end 16.7132 -58.8797) (width 0.1270) (layer "F.Mask") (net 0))
 (segment (start 16.7132 -58.8797) (end 16.7132 -58.8797) (width 0.1270) (layer "F.Mask") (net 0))
 (segment (start 16.7132 -58.8797) (end 16.8148 -58.9610) (width 0.1270) (layer "F.Mask") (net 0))
 (segment (start 16.8148 -58.9610) (end 16.8148 -58.9610) (width 0.1270) (layer "F.Mask") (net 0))
 (segment (start 16.8148 -58.9610) (end 16.8326 -58.9763) (width 0.1270) (layer "F.Mask") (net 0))
 (segment (start 16.8326 -58.9763) (end 16.8326 -58.9763) (width 0.1270) (layer "F.Mask") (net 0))
 (segment (start 16.8326 -58.9763) (end 16.8326 -59.5986) (width 0.1270) (layer "F.Mask") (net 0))
 (segment (start 16.8326 -59.5986) (end 16.8326 -59.5986) (width 0.1270) (layer "F.Mask") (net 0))
 (segment (start 16.8326 -59.5986) (end 16.5202 -59.9110) (width 0.1270) (layer "F.Mask") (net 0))
 (segment (start 16.5202 -59.9110) (end 16.5202 -59.9110) (width 0.1270) (layer "F.Mask") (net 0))
 (segment (start 16.5202 -59.9110) (end 16.5202 -61.0489) (width 0.1270) (layer "F.Mask") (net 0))
 (segment (start 13.8400 -58.7679) (end 13.8400 -58.7679) (width 0.1270) (layer "F.Mask") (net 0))
 (segment (start 13.8400 -58.7679) (end 13.8640 -58.7439) (width 0.1270) (layer "F.Mask") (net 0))
 (segment (start 13.8640 -58.7439) (end 13.8640 -58.7439) (width 0.1270) (layer "F.Mask") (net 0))
 (segment (start 13.8640 -58.7439) (end 13.8640 -57.7999) (width 0.1270) (layer "F.Mask") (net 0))
 (segment (start 11.2243 -57.8079) (end 11.2243 -57.8079) (width 0.1270) (layer "F.Mask") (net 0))
 (segment (start 11.2243 -57.8079) (end 11.2471 -57.8307) (width 0.1270) (layer "F.Mask") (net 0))
 (segment (start 11.2471 -57.8307) (end 11.2471 -57.8307) (width 0.1270) (layer "F.Mask") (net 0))
 (segment (start 11.2471 -57.8307) (end 11.2471 -59.2328) (width 0.1270) (layer "F.Mask") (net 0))
 (segment (start 11.2471 -59.2328) (end 11.2471 -59.2328) (width 0.1270) (layer "F.Mask") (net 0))
 (segment (start 11.2471 -59.2328) (end 12.4638 -60.4469) (width 0.1270) (layer "F.Mask") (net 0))
 (segment (start 12.4638 -60.4469) (end 12.4638 -60.4469) (width 0.1270) (layer "F.Mask") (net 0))
 (segment (start 12.4638 -60.4469) (end 12.4638 -60.9194) (width 0.1270) (layer "F.Mask") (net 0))
 (segment (start 12.3760 -57.9439) (end 12.3760 -57.9439) (width 0.1270) (layer "F.Mask") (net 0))
 (segment (start 12.3760 -57.9439) (end 12.3760 -59.7119) (width 0.1270) (layer "F.Mask") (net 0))
 (segment (start 12.3760 -59.7119) (end 12.3760 -59.7119) (width 0.1270) (layer "F.Mask") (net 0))
 (segment (start 12.3760 -59.7119) (end 13.1760 -60.5119) (width 0.1270) (layer "F.Mask") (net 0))
 (segment (start 13.1760 -60.5119) (end 13.1760 -60.5119) (width 0.1270) (layer "F.Mask") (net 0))
 (segment (start 13.1760 -60.5119) (end 13.1760 -60.6479) (width 0.1270) (layer "F.Mask") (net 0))
 (segment (start 12.8560 -57.9679) (end 12.8560 -57.9679) (width 0.1270) (layer "F.Mask") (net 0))
 (segment (start 12.8560 -57.9679) (end 12.8640 -57.9759) (width 0.1270) (layer "F.Mask") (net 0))
 (segment (start 12.8640 -57.9759) (end 12.8640 -57.9759) (width 0.1270) (layer "F.Mask") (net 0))
 (segment (start 12.8640 -57.9759) (end 12.8640 -59.4479) (width 0.1270) (layer "F.Mask") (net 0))
 (segment (start 14.3760 -57.9679) (end 14.3760 -57.9679) (width 0.1270) (layer "F.Mask") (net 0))
 (segment (start 14.3760 -57.9679) (end 14.4240 -58.0159) (width 0.1270) (layer "F.Mask") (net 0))
 (segment (start 14.4240 -58.0159) (end 14.4240 -58.0159) (width 0.1270) (layer "F.Mask") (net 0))
 (segment (start 14.4240 -58.0159) (end 14.4240 -60.1039) (width 0.1270) (layer "F.Mask") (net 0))
 (segment (start 14.4240 -60.1039) (end 14.4240 -60.1039) (width 0.1270) (layer "F.Mask") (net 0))
 (segment (start 14.4240 -60.1039) (end 14.8400 -60.5199) (width 0.1270) (layer "F.Mask") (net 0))
 (segment (start 14.8400 -60.5199) (end 14.8400 -60.5199) (width 0.1270) (layer "F.Mask") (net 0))
 (segment (start 14.8400 -60.5199) (end 14.8400 -60.8239) (width 0.1270) (layer "F.Mask") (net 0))
 (segment (start 14.8880 -58.0719) (end 14.8880 -58.0719) (width 0.1270) (layer "F.Mask") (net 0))
 (segment (start 14.8880 -58.0719) (end 14.8960 -58.0799) (width 0.1270) (layer "F.Mask") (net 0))
 (segment (start 14.8960 -58.0799) (end 14.8960 -58.0799) (width 0.1270) (layer "F.Mask") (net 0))
 (segment (start 14.8960 -58.0799) (end 14.8960 -59.6879) (width 0.1270) (layer "F.Mask") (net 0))
 (segment (start 15.3600 -58.0559) (end 15.3600 -58.0559) (width 0.1270) (layer "F.Mask") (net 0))
 (segment (start 15.3600 -58.0559) (end 15.3920 -58.0879) (width 0.1270) (layer "F.Mask") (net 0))
 (segment (start 15.3920 -58.0879) (end 15.3920 -58.0879) (width 0.1270) (layer "F.Mask") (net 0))
 (segment (start 15.3920 -58.0879) (end 15.3920 -59.2079) (width 0.1270) (layer "F.Mask") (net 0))
 (segment (start 15.3920 -59.2079) (end 15.3920 -59.2079) (width 0.1270) (layer "F.Mask") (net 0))
 (segment (start 15.3920 -59.2079) (end 15.6240 -59.4399) (width 0.1270) (layer "F.Mask") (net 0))
 (segment (start 15.6240 -59.4399) (end 15.6240 -59.4399) (width 0.1270) (layer "F.Mask") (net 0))
 (segment (start 15.6240 -59.4399) (end 15.6240 -59.4559) (width 0.1270) (layer "F.Mask") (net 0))
 (segment (start 15.6240 -59.4559) (end 15.6240 -59.4559) (width 0.1270) (layer "F.Mask") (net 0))
 (segment (start 15.6240 -59.4559) (end 15.6560 -59.4879) (width 0.1270) (layer "F.Mask") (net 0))
 (segment (start 15.6560 -59.4879) (end 15.6560 -59.4879) (width 0.1270) (layer "F.Mask") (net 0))
 (segment (start 15.6560 -59.4879) (end 15.6560 -61.0719) (width 0.1270) (layer "F.Mask") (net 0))
 (segment (start 15.8320 -57.9679) (end 15.8320 -57.9679) (width 0.1270) (layer "F.Mask") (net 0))
 (segment (start 15.8320 -57.9679) (end 15.8800 -58.0159) (width 0.1270) (layer "F.Mask") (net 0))
 (segment (start 15.8800 -58.0159) (end 15.8800 -58.0159) (width 0.1270) (layer "F.Mask") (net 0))
 (segment (start 15.8800 -58.0159) (end 15.8800 -58.9519) (width 0.1270) (layer "F.Mask") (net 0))
 (segment (start 15.8800 -58.9519) (end 15.8800 -58.9519) (width 0.1270) (layer "F.Mask") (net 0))
 (segment (start 15.8800 -58.9519) (end 16.1520 -59.2239) (width 0.1270) (layer "F.Mask") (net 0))
 (segment (start 16.1520 -59.2239) (end 16.1520 -59.2239) (width 0.1270) (layer "F.Mask") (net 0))
 (segment (start 16.1520 -59.2239) (end 16.1520 -59.2559) (width 0.1270) (layer "F.Mask") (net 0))
 (segment (start 17.3600 -57.8319) (end 17.3600 -57.8319) (width 0.1270) (layer "F.Mask") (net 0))
 (segment (start 17.3600 -57.8319) (end 17.3920 -57.8639) (width 0.1270) (layer "F.Mask") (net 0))
 (segment (start 17.3920 -57.8639) (end 17.3920 -57.8639) (width 0.1270) (layer "F.Mask") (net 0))
 (segment (start 17.3920 -57.8639) (end 17.3920 -60.0319) (width 0.1270) (layer "F.Mask") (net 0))
 (segment (start 17.3920 -60.0319) (end 17.3920 -60.0319) (width 0.1270) (layer "F.Mask") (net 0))
 (segment (start 17.3920 -60.0319) (end 17.2480 -60.1759) (width 0.1270) (layer "F.Mask") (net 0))
 (segment (start 17.2480 -60.1759) (end 17.2480 -60.1759) (width 0.1270) (layer "F.Mask") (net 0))
 (segment (start 17.2480 -60.1759) (end 17.2480 -61.3519) (width 0.1270) (layer "F.Mask") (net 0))
 (segment (start 17.8400 -58.0399) (end 17.8400 -58.0399) (width 0.1270) (layer "F.Mask") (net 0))
 (segment (start 17.8400 -58.0399) (end 17.8800 -58.0799) (width 0.1270) (layer "F.Mask") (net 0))
 (segment (start 17.8800 -58.0799) (end 17.8800 -58.0799) (width 0.1270) (layer "F.Mask") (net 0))
 (segment (start 17.8800 -58.0799) (end 17.8800 -59.3599) (width 0.1270) (layer "F.Mask") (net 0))
 (segment (start 17.8800 -59.3599) (end 17.8800 -59.3599) (width 0.1270) (layer "F.Mask") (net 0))
 (segment (start 17.8800 -59.3599) (end 18.0080 -59.4879) (width 0.1270) (layer "F.Mask") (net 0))
 (segment (start 18.0080 -59.4879) (end 18.0080 -59.4879) (width 0.1270) (layer "F.Mask") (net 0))
 (segment (start 18.0080 -59.4879) (end 18.0080 -59.6559) (width 0.1270) (layer "F.Mask") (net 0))
 (segment (start 19.3523 -58.1762) (end 19.3523 -58.1762) (width 0.1270) (layer "F.Mask") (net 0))
 (segment (start 19.3523 -58.1762) (end 19.3751 -58.1990) (width 0.1270) (layer "F.Mask") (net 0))
 (segment (start 19.3751 -58.1990) (end 19.3751 -58.1990) (width 0.1270) (layer "F.Mask") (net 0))
 (segment (start 19.3751 -58.1990) (end 19.3751 -58.5597) (width 0.1270) (layer "F.Mask") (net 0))
 (segment (start 19.3751 -58.5597) (end 19.3751 -58.5597) (width 0.1270) (layer "F.Mask") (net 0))
 (segment (start 19.3751 -58.5597) (end 19.6317 -58.8162) (width 0.1270) (layer "F.Mask") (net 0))
 (segment (start 19.6317 -58.8162) (end 19.6317 -58.8162) (width 0.1270) (layer "F.Mask") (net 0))
 (segment (start 19.6317 -58.8162) (end 19.6317 -59.2074) (width 0.1270) (layer "F.Mask") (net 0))
 (segment (start 19.6317 -59.2074) (end 19.6317 -59.2074) (width 0.1270) (layer "F.Mask") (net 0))
 (segment (start 19.6317 -59.2074) (end 19.3840 -59.5919) (width 0.1270) (layer "F.Mask") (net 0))
 (segment (start 19.3840 -59.5919) (end 19.3840 -59.5919) (width 0.1270) (layer "F.Mask") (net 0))
 (segment (start 19.3840 -59.5919) (end 19.3827 -59.6087) (width 0.1270) (layer "F.Mask") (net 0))
 (segment (start 19.3827 -59.6087) (end 19.3827 -59.6087) (width 0.1270) (layer "F.Mask") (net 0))
 (segment (start 19.3827 -59.6087) (end 18.8798 -60.1116) (width 0.1270) (layer "F.Mask") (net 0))
 (segment (start 18.8798 -60.1116) (end 18.8798 -60.1116) (width 0.1270) (layer "F.Mask") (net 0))
 (segment (start 18.8798 -60.1116) (end 18.8646 -60.1116) (width 0.1270) (layer "F.Mask") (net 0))
 (segment (start 18.8646 -60.1116) (end 18.8646 -60.1116) (width 0.1270) (layer "F.Mask") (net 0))
 (segment (start 18.8646 -60.1116) (end 18.8646 -61.1276) (width 0.1270) (layer "F.Mask") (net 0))
 (segment (start 18.8560 -57.9359) (end 18.8560 -57.9359) (width 0.1270) (layer "F.Mask") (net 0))
 (segment (start 18.8560 -57.9359) (end 18.8880 -57.9679) (width 0.1270) (layer "F.Mask") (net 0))
 (segment (start 18.8880 -57.9679) (end 18.8880 -57.9679) (width 0.1270) (layer "F.Mask") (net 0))
 (segment (start 18.8880 -57.9679) (end 18.8880 -59.0639) (width 0.1270) (layer "F.Mask") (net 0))
 (segment (start 20.3440 -58.3199) (end 20.3440 -58.3199) (width 0.1270) (layer "F.Mask") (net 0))
 (segment (start 20.3440 -58.3199) (end 20.3760 -58.3519) (width 0.1270) (layer "F.Mask") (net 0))
 (segment (start 20.3760 -58.3519) (end 20.3760 -58.3519) (width 0.1270) (layer "F.Mask") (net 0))
 (segment (start 20.3760 -58.3519) (end 20.3760 -59.2479) (width 0.1270) (layer "F.Mask") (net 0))
 (segment (start 20.3760 -59.2479) (end 20.3760 -59.2479) (width 0.1270) (layer "F.Mask") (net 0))
 (segment (start 20.3760 -59.2479) (end 19.7280 -59.8959) (width 0.1270) (layer "F.Mask") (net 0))
 (segment (start 19.7280 -59.8959) (end 19.7280 -59.8959) (width 0.1270) (layer "F.Mask") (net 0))
 (segment (start 19.7280 -59.8959) (end 19.7280 -59.9039) (width 0.1270) (layer "F.Mask") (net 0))
 (segment (start 19.7280 -59.9039) (end 19.7280 -59.9039) (width 0.1270) (layer "F.Mask") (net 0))
 (segment (start 19.7280 -59.9039) (end 19.6480 -59.9839) (width 0.1270) (layer "F.Mask") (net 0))
 (segment (start 19.6480 -59.9839) (end 19.6480 -59.9839) (width 0.1270) (layer "F.Mask") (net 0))
 (segment (start 19.6480 -59.9839) (end 19.6480 -60.6639) (width 0.1270) (layer "F.Mask") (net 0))
 (gr_line (start 7.0002 -48.0009) (end 7.0002 -48.0009) (layer "Edge.Cuts") (width 0.2540))
 (gr_line (start 7.0002 -48.0009) (end 7.0002 -64.8006) (layer "Edge.Cuts") (width 0.2540))
 (gr_line (start 7.0002 -64.8006) (end 24.7752 -64.8006) (layer "Edge.Cuts") (width 0.2540))
 (gr_line (start 24.7752 -64.8006) (end 24.7752 -48.0009) (layer "Edge.Cuts") (width 0.2540))
 (gr_line (start 24.7752 -48.0009) (end 7.0002 -48.0009) (layer "Edge.Cuts") (width 0.2540)))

